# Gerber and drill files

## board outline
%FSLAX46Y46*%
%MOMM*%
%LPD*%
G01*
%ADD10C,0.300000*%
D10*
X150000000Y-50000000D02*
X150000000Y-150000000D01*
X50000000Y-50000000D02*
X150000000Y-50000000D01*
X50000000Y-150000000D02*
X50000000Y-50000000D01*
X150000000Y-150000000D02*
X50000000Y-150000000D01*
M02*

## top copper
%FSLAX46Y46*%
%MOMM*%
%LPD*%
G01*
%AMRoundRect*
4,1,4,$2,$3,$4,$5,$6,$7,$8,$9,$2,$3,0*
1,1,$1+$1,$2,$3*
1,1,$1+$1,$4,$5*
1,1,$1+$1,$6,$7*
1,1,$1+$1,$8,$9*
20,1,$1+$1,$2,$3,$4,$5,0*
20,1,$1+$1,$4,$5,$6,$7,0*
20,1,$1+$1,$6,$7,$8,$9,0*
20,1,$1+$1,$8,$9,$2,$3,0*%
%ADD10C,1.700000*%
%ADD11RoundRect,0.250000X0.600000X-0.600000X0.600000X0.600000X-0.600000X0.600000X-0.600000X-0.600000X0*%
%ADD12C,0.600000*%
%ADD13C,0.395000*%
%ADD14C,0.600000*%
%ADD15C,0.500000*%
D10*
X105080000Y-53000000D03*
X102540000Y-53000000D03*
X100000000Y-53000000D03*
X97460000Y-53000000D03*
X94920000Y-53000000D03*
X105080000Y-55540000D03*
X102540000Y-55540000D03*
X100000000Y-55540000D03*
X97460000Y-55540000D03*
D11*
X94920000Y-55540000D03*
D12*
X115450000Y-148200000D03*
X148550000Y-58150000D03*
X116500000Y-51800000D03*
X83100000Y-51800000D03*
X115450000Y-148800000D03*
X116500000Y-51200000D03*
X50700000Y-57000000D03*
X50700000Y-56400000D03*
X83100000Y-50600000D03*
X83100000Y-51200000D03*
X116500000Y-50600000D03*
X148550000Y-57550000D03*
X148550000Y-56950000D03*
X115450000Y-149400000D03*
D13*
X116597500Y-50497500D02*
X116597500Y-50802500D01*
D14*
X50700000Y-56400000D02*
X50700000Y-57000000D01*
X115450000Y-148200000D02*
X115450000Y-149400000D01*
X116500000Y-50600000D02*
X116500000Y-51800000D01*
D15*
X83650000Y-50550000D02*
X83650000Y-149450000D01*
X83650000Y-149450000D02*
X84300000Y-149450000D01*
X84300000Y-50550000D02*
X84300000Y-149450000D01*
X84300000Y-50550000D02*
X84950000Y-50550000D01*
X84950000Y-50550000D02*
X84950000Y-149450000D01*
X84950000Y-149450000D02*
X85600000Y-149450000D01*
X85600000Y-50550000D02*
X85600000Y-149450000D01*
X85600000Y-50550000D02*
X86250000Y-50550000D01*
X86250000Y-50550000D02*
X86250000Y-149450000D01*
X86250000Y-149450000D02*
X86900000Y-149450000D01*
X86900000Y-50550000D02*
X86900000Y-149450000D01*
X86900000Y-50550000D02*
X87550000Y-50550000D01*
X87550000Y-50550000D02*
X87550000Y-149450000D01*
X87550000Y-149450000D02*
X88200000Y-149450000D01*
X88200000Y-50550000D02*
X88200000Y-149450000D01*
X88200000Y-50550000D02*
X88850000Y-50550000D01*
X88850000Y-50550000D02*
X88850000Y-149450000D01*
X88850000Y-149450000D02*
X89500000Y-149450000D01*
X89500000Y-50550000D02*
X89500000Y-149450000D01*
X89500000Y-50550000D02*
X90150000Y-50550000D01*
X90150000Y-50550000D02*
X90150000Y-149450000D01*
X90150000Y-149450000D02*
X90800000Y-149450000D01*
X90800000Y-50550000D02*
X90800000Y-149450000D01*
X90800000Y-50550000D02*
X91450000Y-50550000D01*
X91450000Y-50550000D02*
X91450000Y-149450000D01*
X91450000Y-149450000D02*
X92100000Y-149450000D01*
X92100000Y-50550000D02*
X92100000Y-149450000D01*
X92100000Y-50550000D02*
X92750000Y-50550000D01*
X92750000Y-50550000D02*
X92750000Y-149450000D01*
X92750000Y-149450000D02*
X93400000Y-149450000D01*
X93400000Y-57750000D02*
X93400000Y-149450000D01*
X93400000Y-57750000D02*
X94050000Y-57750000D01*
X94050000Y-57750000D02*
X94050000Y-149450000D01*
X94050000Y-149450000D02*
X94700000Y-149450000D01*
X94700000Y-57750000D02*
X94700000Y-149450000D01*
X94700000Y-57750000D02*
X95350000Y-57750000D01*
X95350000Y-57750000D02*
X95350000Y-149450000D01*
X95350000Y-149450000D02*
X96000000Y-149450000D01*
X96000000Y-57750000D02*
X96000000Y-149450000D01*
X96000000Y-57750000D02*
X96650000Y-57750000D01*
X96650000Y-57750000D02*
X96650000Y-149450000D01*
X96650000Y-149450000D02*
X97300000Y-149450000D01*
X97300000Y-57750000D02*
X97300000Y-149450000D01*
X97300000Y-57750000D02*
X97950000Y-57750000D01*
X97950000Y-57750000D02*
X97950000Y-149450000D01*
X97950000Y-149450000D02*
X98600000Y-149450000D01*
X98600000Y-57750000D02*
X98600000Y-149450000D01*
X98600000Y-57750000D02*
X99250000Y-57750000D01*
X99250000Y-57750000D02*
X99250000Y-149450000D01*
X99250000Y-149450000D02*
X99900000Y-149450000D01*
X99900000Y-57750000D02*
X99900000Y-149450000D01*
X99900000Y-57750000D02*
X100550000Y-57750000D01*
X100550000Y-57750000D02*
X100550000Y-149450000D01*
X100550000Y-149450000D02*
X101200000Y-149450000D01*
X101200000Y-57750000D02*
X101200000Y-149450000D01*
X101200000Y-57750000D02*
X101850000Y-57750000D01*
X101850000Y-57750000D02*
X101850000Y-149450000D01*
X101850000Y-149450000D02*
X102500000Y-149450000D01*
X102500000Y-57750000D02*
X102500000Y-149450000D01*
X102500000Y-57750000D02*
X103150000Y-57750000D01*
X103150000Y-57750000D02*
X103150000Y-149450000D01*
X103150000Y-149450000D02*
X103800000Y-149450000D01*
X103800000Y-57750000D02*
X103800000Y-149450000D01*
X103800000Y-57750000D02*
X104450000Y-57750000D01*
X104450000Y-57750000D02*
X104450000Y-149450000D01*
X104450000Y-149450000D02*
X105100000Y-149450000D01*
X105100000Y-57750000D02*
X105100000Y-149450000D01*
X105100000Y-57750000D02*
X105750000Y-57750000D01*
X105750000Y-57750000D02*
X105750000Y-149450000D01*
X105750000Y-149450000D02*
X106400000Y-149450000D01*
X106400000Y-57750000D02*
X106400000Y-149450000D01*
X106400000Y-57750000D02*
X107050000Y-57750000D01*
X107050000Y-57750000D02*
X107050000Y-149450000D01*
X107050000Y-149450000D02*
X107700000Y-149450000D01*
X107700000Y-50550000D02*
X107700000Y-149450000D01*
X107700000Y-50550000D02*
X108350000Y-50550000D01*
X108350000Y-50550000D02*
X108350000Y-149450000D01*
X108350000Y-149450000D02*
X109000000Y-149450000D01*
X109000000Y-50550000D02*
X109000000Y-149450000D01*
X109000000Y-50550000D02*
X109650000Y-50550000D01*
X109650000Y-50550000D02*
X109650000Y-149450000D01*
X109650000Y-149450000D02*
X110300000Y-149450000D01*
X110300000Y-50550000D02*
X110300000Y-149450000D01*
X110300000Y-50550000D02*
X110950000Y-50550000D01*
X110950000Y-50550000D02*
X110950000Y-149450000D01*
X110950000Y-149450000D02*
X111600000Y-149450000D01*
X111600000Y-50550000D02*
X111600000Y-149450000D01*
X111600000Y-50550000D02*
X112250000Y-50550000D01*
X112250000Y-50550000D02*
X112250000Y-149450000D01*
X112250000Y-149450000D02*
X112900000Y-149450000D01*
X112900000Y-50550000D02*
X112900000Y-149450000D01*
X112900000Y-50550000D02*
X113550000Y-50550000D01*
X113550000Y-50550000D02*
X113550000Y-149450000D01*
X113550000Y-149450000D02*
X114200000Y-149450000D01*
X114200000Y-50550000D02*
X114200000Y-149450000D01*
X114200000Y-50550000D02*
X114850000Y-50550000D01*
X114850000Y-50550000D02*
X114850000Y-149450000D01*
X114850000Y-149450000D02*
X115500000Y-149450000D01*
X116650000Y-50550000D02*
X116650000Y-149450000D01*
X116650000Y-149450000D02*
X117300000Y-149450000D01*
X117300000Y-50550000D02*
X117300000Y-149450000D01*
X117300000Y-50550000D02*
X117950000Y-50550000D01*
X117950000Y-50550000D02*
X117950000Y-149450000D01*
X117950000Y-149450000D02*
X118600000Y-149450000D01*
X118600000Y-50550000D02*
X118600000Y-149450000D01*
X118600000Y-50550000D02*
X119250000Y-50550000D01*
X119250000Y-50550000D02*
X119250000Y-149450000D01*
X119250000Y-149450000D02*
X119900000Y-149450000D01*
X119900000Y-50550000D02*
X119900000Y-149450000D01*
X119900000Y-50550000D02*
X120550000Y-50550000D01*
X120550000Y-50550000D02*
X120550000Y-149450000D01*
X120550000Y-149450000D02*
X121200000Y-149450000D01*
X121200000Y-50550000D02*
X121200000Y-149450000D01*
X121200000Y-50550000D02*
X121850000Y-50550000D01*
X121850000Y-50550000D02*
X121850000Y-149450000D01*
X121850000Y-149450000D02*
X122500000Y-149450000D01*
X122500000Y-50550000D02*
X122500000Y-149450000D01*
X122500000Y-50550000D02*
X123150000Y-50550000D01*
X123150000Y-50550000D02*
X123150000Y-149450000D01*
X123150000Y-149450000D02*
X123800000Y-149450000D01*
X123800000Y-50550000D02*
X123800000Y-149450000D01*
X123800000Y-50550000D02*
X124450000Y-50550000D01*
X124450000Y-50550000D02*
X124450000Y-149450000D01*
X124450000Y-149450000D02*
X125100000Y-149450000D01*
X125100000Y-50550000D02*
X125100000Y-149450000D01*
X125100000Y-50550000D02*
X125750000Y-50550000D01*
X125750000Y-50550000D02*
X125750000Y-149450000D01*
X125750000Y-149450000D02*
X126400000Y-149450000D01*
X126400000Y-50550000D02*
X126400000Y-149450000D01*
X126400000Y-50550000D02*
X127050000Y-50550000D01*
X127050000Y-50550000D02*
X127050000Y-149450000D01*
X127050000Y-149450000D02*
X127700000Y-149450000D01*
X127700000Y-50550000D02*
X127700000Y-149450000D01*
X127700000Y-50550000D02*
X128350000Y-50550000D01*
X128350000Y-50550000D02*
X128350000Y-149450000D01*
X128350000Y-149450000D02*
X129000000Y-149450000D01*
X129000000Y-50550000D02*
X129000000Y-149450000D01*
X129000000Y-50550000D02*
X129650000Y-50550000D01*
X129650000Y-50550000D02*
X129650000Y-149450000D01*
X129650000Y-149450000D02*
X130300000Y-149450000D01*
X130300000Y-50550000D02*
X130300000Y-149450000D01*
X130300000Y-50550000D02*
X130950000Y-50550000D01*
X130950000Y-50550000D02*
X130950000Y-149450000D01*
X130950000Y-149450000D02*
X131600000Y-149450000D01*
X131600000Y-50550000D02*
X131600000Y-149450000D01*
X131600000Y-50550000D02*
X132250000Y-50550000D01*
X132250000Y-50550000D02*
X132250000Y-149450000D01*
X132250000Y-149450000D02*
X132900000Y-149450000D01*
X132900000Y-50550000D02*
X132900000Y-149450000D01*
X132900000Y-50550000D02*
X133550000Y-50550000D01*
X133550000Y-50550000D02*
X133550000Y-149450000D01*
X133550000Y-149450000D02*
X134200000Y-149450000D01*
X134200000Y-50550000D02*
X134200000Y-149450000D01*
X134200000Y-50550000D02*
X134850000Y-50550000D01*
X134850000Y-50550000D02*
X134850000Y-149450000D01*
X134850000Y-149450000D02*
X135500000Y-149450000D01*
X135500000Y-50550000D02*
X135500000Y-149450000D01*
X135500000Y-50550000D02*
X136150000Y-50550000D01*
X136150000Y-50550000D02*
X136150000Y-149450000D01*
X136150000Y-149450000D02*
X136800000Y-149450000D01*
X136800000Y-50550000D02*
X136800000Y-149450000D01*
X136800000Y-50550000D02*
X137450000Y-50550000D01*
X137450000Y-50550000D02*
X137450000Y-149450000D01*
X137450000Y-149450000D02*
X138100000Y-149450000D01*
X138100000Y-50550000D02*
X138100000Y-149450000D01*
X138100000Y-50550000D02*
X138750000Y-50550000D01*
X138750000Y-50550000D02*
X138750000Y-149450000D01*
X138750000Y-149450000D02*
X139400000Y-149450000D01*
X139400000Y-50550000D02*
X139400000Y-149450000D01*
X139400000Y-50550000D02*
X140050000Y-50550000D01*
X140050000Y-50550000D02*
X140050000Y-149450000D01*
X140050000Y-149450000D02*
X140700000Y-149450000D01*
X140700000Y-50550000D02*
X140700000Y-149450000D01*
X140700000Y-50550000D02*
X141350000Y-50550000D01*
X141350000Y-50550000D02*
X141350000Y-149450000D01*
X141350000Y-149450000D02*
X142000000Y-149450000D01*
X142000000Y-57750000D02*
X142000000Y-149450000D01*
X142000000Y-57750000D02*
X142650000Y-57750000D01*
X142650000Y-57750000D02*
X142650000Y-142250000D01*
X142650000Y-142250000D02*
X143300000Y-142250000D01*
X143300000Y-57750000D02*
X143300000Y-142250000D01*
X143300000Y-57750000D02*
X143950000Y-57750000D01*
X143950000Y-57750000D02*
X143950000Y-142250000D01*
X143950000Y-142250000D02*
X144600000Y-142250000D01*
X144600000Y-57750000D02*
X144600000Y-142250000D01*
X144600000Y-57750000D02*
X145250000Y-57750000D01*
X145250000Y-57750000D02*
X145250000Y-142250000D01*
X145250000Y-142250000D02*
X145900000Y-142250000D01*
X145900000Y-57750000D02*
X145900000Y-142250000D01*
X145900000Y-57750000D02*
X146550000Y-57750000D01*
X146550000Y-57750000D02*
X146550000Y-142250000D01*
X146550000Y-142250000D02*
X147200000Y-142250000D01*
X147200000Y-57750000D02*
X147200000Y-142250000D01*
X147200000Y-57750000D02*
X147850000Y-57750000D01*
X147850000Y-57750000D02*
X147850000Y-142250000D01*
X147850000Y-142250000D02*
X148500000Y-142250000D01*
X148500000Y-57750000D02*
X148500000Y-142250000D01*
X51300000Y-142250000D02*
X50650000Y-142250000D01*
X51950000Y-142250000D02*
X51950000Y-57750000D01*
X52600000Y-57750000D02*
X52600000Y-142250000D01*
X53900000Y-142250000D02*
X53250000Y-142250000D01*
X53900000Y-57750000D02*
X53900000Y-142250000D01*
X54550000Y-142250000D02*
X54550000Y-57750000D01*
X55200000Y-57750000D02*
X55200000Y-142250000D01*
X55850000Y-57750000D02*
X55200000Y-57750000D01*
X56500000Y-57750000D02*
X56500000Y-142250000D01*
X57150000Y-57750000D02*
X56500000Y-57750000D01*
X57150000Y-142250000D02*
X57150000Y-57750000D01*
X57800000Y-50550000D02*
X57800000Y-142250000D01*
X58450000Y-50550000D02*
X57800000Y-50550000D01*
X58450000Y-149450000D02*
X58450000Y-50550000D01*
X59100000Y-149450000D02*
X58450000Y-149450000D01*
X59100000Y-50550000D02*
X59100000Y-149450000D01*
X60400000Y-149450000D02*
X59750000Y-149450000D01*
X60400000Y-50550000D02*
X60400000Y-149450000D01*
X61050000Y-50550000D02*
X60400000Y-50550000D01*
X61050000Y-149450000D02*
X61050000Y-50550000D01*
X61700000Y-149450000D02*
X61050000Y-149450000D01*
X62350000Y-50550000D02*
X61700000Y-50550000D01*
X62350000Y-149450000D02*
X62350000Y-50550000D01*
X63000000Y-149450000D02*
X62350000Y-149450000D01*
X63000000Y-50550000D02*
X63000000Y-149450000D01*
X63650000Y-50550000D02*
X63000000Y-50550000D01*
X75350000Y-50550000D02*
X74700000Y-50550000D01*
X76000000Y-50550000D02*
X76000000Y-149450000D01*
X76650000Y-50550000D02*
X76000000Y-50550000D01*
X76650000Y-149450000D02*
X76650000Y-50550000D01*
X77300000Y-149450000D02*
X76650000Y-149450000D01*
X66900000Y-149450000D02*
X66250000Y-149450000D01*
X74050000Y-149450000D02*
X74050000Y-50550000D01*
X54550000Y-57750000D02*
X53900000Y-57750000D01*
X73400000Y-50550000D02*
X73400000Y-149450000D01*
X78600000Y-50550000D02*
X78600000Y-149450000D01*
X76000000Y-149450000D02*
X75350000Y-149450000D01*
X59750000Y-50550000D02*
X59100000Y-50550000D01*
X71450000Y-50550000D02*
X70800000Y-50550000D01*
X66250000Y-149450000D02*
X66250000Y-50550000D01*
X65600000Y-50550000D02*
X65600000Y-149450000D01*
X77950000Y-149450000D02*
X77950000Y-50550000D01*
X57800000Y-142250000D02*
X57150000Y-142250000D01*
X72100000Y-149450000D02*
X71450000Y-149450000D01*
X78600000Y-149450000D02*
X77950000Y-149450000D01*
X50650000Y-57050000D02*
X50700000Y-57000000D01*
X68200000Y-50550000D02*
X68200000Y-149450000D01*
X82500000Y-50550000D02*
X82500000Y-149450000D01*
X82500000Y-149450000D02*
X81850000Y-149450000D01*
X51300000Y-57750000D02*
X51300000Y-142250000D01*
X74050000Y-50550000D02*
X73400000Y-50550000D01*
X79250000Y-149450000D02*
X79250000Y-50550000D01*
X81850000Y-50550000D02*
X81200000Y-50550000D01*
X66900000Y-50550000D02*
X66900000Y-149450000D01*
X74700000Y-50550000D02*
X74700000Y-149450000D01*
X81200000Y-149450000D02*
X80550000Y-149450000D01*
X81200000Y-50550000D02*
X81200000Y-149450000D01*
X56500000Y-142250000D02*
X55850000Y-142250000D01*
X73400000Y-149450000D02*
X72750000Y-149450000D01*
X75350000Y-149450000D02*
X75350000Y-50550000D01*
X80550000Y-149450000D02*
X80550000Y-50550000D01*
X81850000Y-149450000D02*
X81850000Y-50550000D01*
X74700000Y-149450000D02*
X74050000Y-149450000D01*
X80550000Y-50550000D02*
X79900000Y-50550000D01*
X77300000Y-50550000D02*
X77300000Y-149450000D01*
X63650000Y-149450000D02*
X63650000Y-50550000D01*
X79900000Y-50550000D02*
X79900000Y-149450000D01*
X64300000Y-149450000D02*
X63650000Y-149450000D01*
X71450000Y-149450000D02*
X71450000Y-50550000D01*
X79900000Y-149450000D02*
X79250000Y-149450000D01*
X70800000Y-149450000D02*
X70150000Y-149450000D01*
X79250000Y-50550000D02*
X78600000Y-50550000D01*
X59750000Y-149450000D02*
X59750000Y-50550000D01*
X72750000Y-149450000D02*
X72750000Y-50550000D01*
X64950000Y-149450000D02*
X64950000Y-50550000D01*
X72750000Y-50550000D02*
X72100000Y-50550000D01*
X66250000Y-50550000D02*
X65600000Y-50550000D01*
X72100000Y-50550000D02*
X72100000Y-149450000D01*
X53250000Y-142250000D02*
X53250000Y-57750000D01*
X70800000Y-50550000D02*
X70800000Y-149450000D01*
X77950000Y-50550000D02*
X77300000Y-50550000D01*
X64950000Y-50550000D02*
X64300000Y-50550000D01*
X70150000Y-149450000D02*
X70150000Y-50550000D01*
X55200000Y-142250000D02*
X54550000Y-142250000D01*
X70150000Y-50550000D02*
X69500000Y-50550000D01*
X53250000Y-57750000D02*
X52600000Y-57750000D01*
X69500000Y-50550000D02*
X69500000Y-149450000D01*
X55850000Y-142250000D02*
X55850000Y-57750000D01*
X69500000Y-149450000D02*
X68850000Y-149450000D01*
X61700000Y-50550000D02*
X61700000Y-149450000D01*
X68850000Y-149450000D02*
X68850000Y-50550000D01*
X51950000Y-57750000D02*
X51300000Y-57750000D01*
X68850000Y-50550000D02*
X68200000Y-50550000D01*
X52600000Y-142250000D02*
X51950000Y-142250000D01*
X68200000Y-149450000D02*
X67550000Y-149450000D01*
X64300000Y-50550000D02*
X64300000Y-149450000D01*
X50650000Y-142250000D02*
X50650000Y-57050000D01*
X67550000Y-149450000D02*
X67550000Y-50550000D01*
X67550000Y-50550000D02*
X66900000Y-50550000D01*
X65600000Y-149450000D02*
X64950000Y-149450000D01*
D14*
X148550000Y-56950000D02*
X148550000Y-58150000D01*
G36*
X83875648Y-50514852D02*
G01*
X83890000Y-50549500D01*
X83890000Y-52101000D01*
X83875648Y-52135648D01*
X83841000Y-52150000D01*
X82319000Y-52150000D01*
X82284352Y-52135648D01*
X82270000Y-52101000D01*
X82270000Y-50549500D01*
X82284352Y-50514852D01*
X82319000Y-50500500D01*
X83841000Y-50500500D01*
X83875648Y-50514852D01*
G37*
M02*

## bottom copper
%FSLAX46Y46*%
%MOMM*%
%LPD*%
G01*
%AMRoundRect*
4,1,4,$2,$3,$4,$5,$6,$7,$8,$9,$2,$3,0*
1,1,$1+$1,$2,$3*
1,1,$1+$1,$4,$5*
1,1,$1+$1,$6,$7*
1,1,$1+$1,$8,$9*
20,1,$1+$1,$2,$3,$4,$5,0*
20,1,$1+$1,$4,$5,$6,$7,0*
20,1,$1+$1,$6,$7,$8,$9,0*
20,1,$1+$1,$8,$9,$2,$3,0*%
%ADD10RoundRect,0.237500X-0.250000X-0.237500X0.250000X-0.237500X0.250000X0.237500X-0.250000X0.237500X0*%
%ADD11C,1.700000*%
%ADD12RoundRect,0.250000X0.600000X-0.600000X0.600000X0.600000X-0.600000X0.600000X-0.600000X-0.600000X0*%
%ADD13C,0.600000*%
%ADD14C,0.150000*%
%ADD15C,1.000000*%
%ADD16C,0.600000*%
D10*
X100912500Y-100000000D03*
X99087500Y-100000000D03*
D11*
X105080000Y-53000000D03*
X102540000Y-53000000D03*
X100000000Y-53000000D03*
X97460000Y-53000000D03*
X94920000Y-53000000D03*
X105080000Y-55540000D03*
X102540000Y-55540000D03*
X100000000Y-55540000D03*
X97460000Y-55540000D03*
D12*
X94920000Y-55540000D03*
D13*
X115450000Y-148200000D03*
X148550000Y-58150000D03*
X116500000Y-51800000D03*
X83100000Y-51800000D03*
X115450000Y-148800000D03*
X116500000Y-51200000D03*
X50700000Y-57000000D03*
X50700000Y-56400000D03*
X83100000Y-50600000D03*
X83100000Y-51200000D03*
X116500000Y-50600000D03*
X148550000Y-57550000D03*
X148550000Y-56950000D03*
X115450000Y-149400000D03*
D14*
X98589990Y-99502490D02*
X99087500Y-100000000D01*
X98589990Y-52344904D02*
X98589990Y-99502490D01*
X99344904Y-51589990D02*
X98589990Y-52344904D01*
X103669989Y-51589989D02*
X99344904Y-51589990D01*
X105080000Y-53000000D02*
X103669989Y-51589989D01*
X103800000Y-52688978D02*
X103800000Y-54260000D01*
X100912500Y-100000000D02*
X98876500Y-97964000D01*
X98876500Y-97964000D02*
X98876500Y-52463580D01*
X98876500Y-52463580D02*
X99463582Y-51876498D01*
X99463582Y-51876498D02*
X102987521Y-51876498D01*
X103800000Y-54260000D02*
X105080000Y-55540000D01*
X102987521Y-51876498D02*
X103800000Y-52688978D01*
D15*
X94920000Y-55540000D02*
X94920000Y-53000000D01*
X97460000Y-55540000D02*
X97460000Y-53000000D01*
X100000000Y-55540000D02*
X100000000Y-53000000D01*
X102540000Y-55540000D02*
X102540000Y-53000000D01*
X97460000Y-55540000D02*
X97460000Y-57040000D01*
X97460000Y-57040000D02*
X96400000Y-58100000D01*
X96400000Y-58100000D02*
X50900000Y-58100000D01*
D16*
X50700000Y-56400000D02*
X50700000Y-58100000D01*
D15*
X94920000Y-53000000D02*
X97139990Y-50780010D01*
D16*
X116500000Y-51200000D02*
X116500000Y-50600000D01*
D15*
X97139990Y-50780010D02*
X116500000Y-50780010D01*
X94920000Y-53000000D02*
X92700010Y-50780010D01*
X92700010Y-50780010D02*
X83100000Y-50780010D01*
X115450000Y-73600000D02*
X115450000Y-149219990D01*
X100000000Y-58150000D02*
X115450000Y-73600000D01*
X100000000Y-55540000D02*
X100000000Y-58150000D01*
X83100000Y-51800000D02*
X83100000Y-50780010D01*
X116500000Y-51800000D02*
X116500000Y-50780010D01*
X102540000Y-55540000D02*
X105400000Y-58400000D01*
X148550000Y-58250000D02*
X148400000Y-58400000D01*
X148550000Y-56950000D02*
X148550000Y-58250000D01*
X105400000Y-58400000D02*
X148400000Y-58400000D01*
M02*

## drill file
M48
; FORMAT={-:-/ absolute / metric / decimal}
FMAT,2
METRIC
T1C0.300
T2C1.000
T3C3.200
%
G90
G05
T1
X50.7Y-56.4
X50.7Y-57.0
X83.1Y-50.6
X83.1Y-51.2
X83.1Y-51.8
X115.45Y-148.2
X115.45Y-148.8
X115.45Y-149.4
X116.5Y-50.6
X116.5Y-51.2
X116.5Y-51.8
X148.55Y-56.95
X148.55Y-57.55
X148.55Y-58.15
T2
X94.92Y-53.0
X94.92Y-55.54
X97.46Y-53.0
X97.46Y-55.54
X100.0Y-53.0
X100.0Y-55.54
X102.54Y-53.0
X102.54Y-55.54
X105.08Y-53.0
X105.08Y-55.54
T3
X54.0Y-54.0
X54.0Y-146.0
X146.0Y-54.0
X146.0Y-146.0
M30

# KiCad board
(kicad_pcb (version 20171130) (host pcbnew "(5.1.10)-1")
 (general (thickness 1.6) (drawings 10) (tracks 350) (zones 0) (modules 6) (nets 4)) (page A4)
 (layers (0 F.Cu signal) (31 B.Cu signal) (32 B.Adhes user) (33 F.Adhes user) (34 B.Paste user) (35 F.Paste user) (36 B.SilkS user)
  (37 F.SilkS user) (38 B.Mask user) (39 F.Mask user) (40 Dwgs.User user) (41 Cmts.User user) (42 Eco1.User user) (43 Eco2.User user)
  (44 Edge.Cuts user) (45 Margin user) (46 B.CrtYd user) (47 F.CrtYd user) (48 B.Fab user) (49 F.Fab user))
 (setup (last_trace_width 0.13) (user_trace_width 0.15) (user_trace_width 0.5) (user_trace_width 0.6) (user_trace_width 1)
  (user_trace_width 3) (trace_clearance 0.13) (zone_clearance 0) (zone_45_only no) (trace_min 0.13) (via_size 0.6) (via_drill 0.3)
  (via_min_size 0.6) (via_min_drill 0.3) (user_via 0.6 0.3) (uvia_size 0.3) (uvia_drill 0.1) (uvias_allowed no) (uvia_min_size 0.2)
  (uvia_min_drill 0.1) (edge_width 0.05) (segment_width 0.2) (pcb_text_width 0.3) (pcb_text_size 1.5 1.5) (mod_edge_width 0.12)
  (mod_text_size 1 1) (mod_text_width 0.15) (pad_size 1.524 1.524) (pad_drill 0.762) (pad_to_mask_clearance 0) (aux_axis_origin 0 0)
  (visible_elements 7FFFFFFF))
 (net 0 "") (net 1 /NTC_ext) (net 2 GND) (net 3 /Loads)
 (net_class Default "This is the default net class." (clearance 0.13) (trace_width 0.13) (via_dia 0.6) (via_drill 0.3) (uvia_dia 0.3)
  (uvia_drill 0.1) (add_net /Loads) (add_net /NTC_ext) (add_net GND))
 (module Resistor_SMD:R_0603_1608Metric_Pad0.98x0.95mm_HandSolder (layer B.Cu) (at 100 100)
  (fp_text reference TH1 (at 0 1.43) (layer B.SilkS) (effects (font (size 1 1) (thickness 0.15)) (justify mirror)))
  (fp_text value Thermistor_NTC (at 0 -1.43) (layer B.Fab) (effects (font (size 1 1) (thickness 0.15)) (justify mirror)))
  (pad 2 smd roundrect (at 0.9125 0) (size 0.975 0.95) (layers B.Cu B.Paste B.Mask) (roundrect_rratio 0.25) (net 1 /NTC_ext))
  (pad 1 smd roundrect (at -0.9125 0) (size 0.975 0.95) (layers B.Cu B.Paste B.Mask) (roundrect_rratio 0.25) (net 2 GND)))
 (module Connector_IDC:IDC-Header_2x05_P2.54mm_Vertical (layer F.Cu) (at 94.92 55.54 90)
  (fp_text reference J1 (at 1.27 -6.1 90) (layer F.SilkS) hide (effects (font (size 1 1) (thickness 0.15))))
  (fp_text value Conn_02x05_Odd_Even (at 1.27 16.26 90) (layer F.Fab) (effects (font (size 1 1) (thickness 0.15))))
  (pad 10 thru_hole circle (at 2.54 10.16 90) (size 1.7 1.7) (drill 1) (layers *.Cu *.Mask) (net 2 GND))
  (pad 8 thru_hole circle (at 2.54 7.62 90) (size 1.7 1.7) (drill 1) (layers *.Cu *.Mask) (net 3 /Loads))
  (pad 6 thru_hole circle (at 2.54 5.08 90) (size 1.7 1.7) (drill 1) (layers *.Cu *.Mask) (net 3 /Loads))
  (pad 4 thru_hole circle (at 2.54 2.54 90) (size 1.7 1.7) (drill 1) (layers *.Cu *.Mask) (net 3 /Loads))
  (pad 2 thru_hole circle (at 2.54 0 90) (size 1.7 1.7) (drill 1) (layers *.Cu *.Mask) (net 3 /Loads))
  (pad 9 thru_hole circle (at 0 10.16 90) (size 1.7 1.7) (drill 1) (layers *.Cu *.Mask) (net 1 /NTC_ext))
  (pad 7 thru_hole circle (at 0 7.62 90) (size 1.7 1.7) (drill 1) (layers *.Cu *.Mask) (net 3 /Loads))
  (pad 5 thru_hole circle (at 0 5.08 90) (size 1.7 1.7) (drill 1) (layers *.Cu *.Mask) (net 3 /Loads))
  (pad 3 thru_hole circle (at 0 2.54 90) (size 1.7 1.7) (drill 1) (layers *.Cu *.Mask) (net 3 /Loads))
  (pad 1 thru_hole roundrect (at 0 0 90) (size 1.7 1.7) (drill 1) (layers *.Cu *.Mask) (roundrect_rratio 0.1470588235294118) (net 3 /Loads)))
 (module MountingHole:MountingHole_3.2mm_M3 (layer F.Cu) (at 146 146)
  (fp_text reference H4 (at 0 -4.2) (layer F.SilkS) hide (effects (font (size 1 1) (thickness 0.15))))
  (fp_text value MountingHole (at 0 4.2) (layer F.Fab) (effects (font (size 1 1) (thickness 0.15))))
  (pad 1 np_thru_hole circle (at 0 0) (size 3.2 3.2) (drill 3.2) (layers *.Cu *.Mask)))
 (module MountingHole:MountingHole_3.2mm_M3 (layer F.Cu) (at 54 146)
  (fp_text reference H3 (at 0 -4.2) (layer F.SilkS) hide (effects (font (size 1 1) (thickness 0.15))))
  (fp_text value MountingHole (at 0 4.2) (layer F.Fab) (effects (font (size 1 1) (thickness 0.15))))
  (pad 1 np_thru_hole circle (at 0 0) (size 3.2 3.2) (drill 3.2) (layers *.Cu *.Mask)))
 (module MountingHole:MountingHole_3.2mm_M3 (layer F.Cu) (at 146 54)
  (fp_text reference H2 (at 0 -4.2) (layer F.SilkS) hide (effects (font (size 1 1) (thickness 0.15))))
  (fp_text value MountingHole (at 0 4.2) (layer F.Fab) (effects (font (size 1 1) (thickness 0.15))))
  (pad 1 np_thru_hole circle (at 0 0) (size 3.2 3.2) (drill 3.2) (layers *.Cu *.Mask)))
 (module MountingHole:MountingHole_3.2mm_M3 (layer F.Cu) (at 54 54)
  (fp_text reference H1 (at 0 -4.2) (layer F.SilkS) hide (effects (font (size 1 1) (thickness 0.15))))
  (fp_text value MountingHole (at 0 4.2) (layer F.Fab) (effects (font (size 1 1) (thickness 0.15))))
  (pad 1 np_thru_hole circle (at 0 0) (size 3.2 3.2) (drill 3.2) (layers *.Cu *.Mask)))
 (gr_line (start 150 50) (end 150 150) (layer Edge.Cuts) (width 0.3))
 (gr_line (start 50 50) (end 150 50) (layer Edge.Cuts) (width 0.3))
 (gr_line (start 50 150) (end 50 50) (layer Edge.Cuts) (width 0.3))
 (gr_line (start 150 150) (end 50 150) (layer Edge.Cuts) (width 0.3))
 (segment (start 98.58999 99.50249) (end 99.0875 100) (width 0.15) (layer B.Cu) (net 2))
 (segment (start 98.58999 52.344904) (end 98.58999 99.50249) (width 0.15) (layer B.Cu) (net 2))
 (segment (start 99.344904 51.58999) (end 98.58999 52.344904) (width 0.15) (layer B.Cu) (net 2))
 (segment (start 103.669989 51.589989) (end 99.344904 51.58999) (width 0.15) (layer B.Cu) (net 2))
 (segment (start 105.08 53) (end 103.669989 51.589989) (width 0.15) (layer B.Cu) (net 2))
 (segment (start 103.8 52.688978) (end 103.8 54.26) (width 0.15) (layer B.Cu) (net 1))
 (segment (start 100.9125 100) (end 98.8765 97.964) (width 0.15) (layer B.Cu) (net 1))
 (segment (start 98.8765 97.964) (end 98.8765 52.46358) (width 0.15) (layer B.Cu) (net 1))
 (segment (start 98.8765 52.46358) (end 99.463582 51.876498) (width 0.15) (layer B.Cu) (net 1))
 (segment (start 99.463582 51.876498) (end 102.987521 51.876498) (width 0.15) (layer B.Cu) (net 1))
 (segment (start 103.8 54.26) (end 105.08 55.54) (width 0.15) (layer B.Cu) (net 1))
 (segment (start 102.987521 51.876498) (end 103.8 52.688978) (width 0.15) (layer B.Cu) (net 1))
 (via (at 115.45 148.2) (size 0.6) (drill 0.3) (layers F.Cu B.Cu) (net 3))
 (via (at 148.55 58.15) (size 0.6) (drill 0.3) (layers F.Cu B.Cu) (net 3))
 (via (at 116.5 51.8) (size 0.6) (drill 0.3) (layers F.Cu B.Cu) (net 3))
 (via (at 83.1 51.8) (size 0.6) (drill 0.3) (layers F.Cu B.Cu) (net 3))
 (via (at 115.45 148.8) (size 0.6) (drill 0.3) (layers F.Cu B.Cu) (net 3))
 (via (at 116.5 51.2) (size 0.6) (drill 0.3) (layers F.Cu B.Cu) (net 3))
 (via (at 50.7 57) (size 0.6) (drill 0.3) (layers F.Cu B.Cu) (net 3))
 (via (at 50.7 56.4) (size 0.6) (drill 0.3) (layers F.Cu B.Cu) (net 3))
 (segment (start 94.92 55.54) (end 94.92 53) (width 1) (layer B.Cu) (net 3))
 (segment (start 97.46 55.54) (end 97.46 53) (width 1) (layer B.Cu) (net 3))
 (segment (start 100 55.54) (end 100 53) (width 1) (layer B.Cu) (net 3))
 (segment (start 102.54 55.54) (end 102.54 53) (width 1) (layer B.Cu) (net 3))
 (segment (start 116.5975 50.4975) (end 116.5975 50.8025) (width 0.395) (layer F.Cu) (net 3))
 (via (at 83.1 50.6) (size 0.6) (drill 0.3) (layers F.Cu B.Cu) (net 3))
 (via (at 83.1 51.2) (size 0.6) (drill 0.3) (layers F.Cu B.Cu) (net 3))
 (segment (start 97.46 55.54) (end 97.46 57.04) (width 1) (layer B.Cu) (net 3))
 (segment (start 97.46 57.04) (end 96.4 58.1) (width 1) (layer B.Cu) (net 3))
 (segment (start 96.4 58.1) (end 50.9 58.1) (width 1) (layer B.Cu) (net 3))
 (segment (start 50.7 56.4) (end 50.7 58.1) (width 0.6) (layer B.Cu) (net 3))
 (segment (start 50.7 56.4) (end 50.7 57) (width 0.6) (layer F.Cu) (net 3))
 (via (at 116.5 50.6) (size 0.6) (drill 0.3) (layers F.Cu B.Cu) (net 3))
 (segment (start 94.92 53) (end 97.13999 50.78001) (width 1) (layer B.Cu) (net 3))
 (segment (start 116.5 51.2) (end 116.5 50.6) (width 0.6) (layer B.Cu) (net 3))
 (segment (start 97.13999 50.78001) (end 116.5 50.78001) (width 1) (layer B.Cu) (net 3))
 (segment (start 94.92 53) (end 92.70001 50.78001) (width 1) (layer B.Cu) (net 3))
 (segment (start 92.70001 50.78001) (end 83.1 50.78001) (width 1) (layer B.Cu) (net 3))
 (via (at 148.55 57.55) (size 0.6) (drill 0.3) (layers F.Cu B.Cu) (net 3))
 (via (at 148.55 56.95) (size 0.6) (drill 0.3) (layers F.Cu B.Cu) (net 3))
 (via (at 115.45 149.4) (size 0.6) (drill 0.3) (layers F.Cu B.Cu) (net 3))
 (segment (start 115.45 73.6) (end 115.45 149.21999) (width 1) (layer B.Cu) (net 3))
 (segment (start 100 58.15) (end 115.45 73.6) (width 1) (layer B.Cu) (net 3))
 (segment (start 100 55.54) (end 100 58.15) (width 1) (layer B.Cu) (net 3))
 (segment (start 83.1 51.8) (end 83.1 50.78001) (width 1) (layer B.Cu) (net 3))
 (segment (start 116.5 51.8) (end 116.5 50.78001) (width 1) (layer B.Cu) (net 3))
 (segment (start 102.54 55.54) (end 105.4 58.4) (width 1) (layer B.Cu) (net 3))
 (segment (start 115.45 148.2) (end 115.45 149.4) (width 0.6) (layer F.Cu) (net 3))
 (segment (start 116.5 50.6) (end 116.5 51.8) (width 0.6) (layer F.Cu) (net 3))
 (segment (start 83.65 50.55) (end 83.65 149.45) (width 0.5) (layer F.Cu) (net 3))
 (segment (start 83.65 149.45) (end 84.3 149.45) (width 0.5) (layer F.Cu) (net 3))
 (segment (start 84.3 50.55) (end 84.3 149.45) (width 0.5) (layer F.Cu) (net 3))
 (segment (start 84.3 50.55) (end 84.95 50.55) (width 0.5) (layer F.Cu) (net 3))
 (segment (start 84.95 50.55) (end 84.95 149.45) (width 0.5) (layer F.Cu) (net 3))
 (segment (start 84.95 149.45) (end 85.6 149.45) (width 0.5) (layer F.Cu) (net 3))
 (segment (start 85.6 50.55) (end 85.6 149.45) (width 0.5) (layer F.Cu) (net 3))
 (segment (start 85.6 50.55) (end 86.25 50.55) (width 0.5) (layer F.Cu) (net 3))
 (segment (start 86.25 50.55) (end 86.25 149.45) (width 0.5) (layer F.Cu) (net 3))
 (segment (start 86.25 149.45) (end 86.9 149.45) (width 0.5) (layer F.Cu) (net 3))
 (segment (start 86.9 50.55) (end 86.9 149.45) (width 0.5) (layer F.Cu) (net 3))
 (segment (start 86.9 50.55) (end 87.55 50.55) (width 0.5) (layer F.Cu) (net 3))
 (segment (start 87.55 50.55) (end 87.55 149.45) (width 0.5) (layer F.Cu) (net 3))
 (segment (start 87.55 149.45) (end 88.2 149.45) (width 0.5) (layer F.Cu) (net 3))
 (segment (start 88.2 50.55) (end 88.2 149.45) (width 0.5) (layer F.Cu) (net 3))
 (segment (start 88.2 50.55) (end 88.85 50.55) (width 0.5) (layer F.Cu) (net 3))
 (segment (start 88.85 50.55) (end 88.85 149.45) (width 0.5) (layer F.Cu) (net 3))
 (segment (start 88.85 149.45) (end 89.5 149.45) (width 0.5) (layer F.Cu) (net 3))
 (segment (start 89.5 50.55) (end 89.5 149.45) (width 0.5) (layer F.Cu) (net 3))
 (segment (start 89.5 50.55) (end 90.15 50.55) (width 0.5) (layer F.Cu) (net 3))
 (segment (start 90.15 50.55) (end 90.15 149.45) (width 0.5) (layer F.Cu) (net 3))
 (segment (start 90.15 149.45) (end 90.8 149.45) (width 0.5) (layer F.Cu) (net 3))
 (segment (start 90.8 50.55) (end 90.8 149.45) (width 0.5) (layer F.Cu) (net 3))
 (segment (start 90.8 50.55) (end 91.45 50.55) (width 0.5) (layer F.Cu) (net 3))
 (segment (start 91.45 50.55) (end 91.45 149.45) (width 0.5) (layer F.Cu) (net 3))
 (segment (start 91.45 149.45) (end 92.1 149.45) (width 0.5) (layer F.Cu) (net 3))
 (segment (start 92.1 50.55) (end 92.1 149.45) (width 0.5) (layer F.Cu) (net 3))
 (segment (start 92.1 50.55) (end 92.75 50.55) (width 0.5) (layer F.Cu) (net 3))
 (segment (start 92.75 50.55) (end 92.75 149.45) (width 0.5) (layer F.Cu) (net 3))
 (segment (start 92.75 149.45) (end 93.4 149.45) (width 0.5) (layer F.Cu) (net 3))
 (segment (start 93.4 57.75) (end 93.4 149.45) (width 0.5) (layer F.Cu) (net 3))
 (segment (start 93.4 57.75) (end 94.05 57.75) (width 0.5) (layer F.Cu) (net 3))
 (segment (start 94.05 57.75) (end 94.05 149.45) (width 0.5) (layer F.Cu) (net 3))
 (segment (start 94.05 149.45) (end 94.7 149.45) (width 0.5) (layer F.Cu) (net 3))
 (segment (start 94.7 57.75) (end 94.7 149.45) (width 0.5) (layer F.Cu) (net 3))
 (segment (start 94.7 57.75) (end 95.35 57.75) (width 0.5) (layer F.Cu) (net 3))
 (segment (start 95.35 57.75) (end 95.35 149.45) (width 0.5) (layer F.Cu) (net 3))
 (segment (start 95.35 149.45) (end 96 149.45) (width 0.5) (layer F.Cu) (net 3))
 (segment (start 96 57.75) (end 96 149.45) (width 0.5) (layer F.Cu) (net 3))
 (segment (start 96 57.75) (end 96.65 57.75) (width 0.5) (layer F.Cu) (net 3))
 (segment (start 96.65 57.75) (end 96.65 149.45) (width 0.5) (layer F.Cu) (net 3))
 (segment (start 96.65 149.45) (end 97.3 149.45) (width 0.5) (layer F.Cu) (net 3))
 (segment (start 97.3 57.75) (end 97.3 149.45) (width 0.5) (layer F.Cu) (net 3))
 (segment (start 97.3 57.75) (end 97.95 57.75) (width 0.5) (layer F.Cu) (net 3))
 (segment (start 97.95 57.75) (end 97.95 149.45) (width 0.5) (layer F.Cu) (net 3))
 (segment (start 97.95 149.45) (end 98.6 149.45) (width 0.5) (layer F.Cu) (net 3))
 (segment (start 98.6 57.75) (end 98.6 149.45) (width 0.5) (layer F.Cu) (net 3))
 (segment (start 98.6 57.75) (end 99.25 57.75) (width 0.5) (layer F.Cu) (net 3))
 (segment (start 99.25 57.75) (end 99.25 149.45) (width 0.5) (layer F.Cu) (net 3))
 (segment (start 99.25 149.45) (end 99.9 149.45) (width 0.5) (layer F.Cu) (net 3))
 (segment (start 99.9 57.75) (end 99.9 149.45) (width 0.5) (layer F.Cu) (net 3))
 (segment (start 99.9 57.75) (end 100.55 57.75) (width 0.5) (layer F.Cu) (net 3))
 (segment (start 100.55 57.75) (end 100.55 149.45) (width 0.5) (layer F.Cu) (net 3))
 (segment (start 100.55 149.45) (end 101.2 149.45) (width 0.5) (layer F.Cu) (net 3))
 (segment (start 101.2 57.75) (end 101.2 149.45) (width 0.5) (layer F.Cu) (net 3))
 (segment (start 101.2 57.75) (end 101.85 57.75) (width 0.5) (layer F.Cu) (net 3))
 (segment (start 101.85 57.75) (end 101.85 149.45) (width 0.5) (layer F.Cu) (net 3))
 (segment (start 101.85 149.45) (end 102.5 149.45) (width 0.5) (layer F.Cu) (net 3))
 (segment (start 102.5 57.75) (end 102.5 149.45) (width 0.5) (layer F.Cu) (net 3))
 (segment (start 102.5 57.75) (end 103.15 57.75) (width 0.5) (layer F.Cu) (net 3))
 (segment (start 103.15 57.75) (end 103.15 149.45) (width 0.5) (layer F.Cu) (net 3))
 (segment (start 103.15 149.45) (end 103.8 149.45) (width 0.5) (layer F.Cu) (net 3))
 (segment (start 103.8 57.75) (end 103.8 149.45) (width 0.5) (layer F.Cu) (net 3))
 (segment (start 103.8 57.75) (end 104.45 57.75) (width 0.5) (layer F.Cu) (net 3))
 (segment (start 104.45 57.75) (end 104.45 149.45) (width 0.5) (layer F.Cu) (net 3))
 (segment (start 104.45 149.45) (end 105.1 149.45) (width 0.5) (layer F.Cu) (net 3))
 (segment (start 105.1 57.75) (end 105.1 149.45) (width 0.5) (layer F.Cu) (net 3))
 (segment (start 105.1 57.75) (end 105.75 57.75) (width 0.5) (layer F.Cu) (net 3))
 (segment (start 105.75 57.75) (end 105.75 149.45) (width 0.5) (layer F.Cu) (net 3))
 (segment (start 105.75 149.45) (end 106.4 149.45) (width 0.5) (layer F.Cu) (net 3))
 (segment (start 106.4 57.75) (end 106.4 149.45) (width 0.5) (layer F.Cu) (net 3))
 (segment (start 106.4 57.75) (end 107.05 57.75) (width 0.5) (layer F.Cu) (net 3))
 (segment (start 107.05 57.75) (end 107.05 149.45) (width 0.5) (layer F.Cu) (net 3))
 (segment (start 107.05 149.45) (end 107.7 149.45) (width 0.5) (layer F.Cu) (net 3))
 (segment (start 107.7 50.55) (end 107.7 149.45) (width 0.5) (layer F.Cu) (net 3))
 (segment (start 107.7 50.55) (end 108.35 50.55) (width 0.5) (layer F.Cu) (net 3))
 (segment (start 108.35 50.55) (end 108.35 149.45) (width 0.5) (layer F.Cu) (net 3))
 (segment (start 108.35 149.45) (end 109 149.45) (width 0.5) (layer F.Cu) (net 3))
 (segment (start 109 50.55) (end 109 149.45) (width 0.5) (layer F.Cu) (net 3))
 (segment (start 109 50.55) (end 109.65 50.55) (width 0.5) (layer F.Cu) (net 3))
 (segment (start 109.65 50.55) (end 109.65 149.45) (width 0.5) (layer F.Cu) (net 3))
 (segment (start 109.65 149.45) (end 110.3 149.45) (width 0.5) (layer F.Cu) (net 3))
 (segment (start 110.3 50.55) (end 110.3 149.45) (width 0.5) (layer F.Cu) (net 3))
 (segment (start 110.3 50.55) (end 110.95 50.55) (width 0.5) (layer F.Cu) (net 3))
 (segment (start 110.95 50.55) (end 110.95 149.45) (width 0.5) (layer F.Cu) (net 3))
 (segment (start 110.95 149.45) (end 111.6 149.45) (width 0.5) (layer F.Cu) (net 3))
 (segment (start 111.6 50.55) (end 111.6 149.45) (width 0.5) (layer F.Cu) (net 3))
 (segment (start 111.6 50.55) (end 112.25 50.55) (width 0.5) (layer F.Cu) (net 3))
 (segment (start 112.25 50.55) (end 112.25 149.45) (width 0.5) (layer F.Cu) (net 3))
 (segment (start 112.25 149.45) (end 112.9 149.45) (width 0.5) (layer F.Cu) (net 3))
 (segment (start 112.9 50.55) (end 112.9 149.45) (width 0.5) (layer F.Cu) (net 3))
 (segment (start 112.9 50.55) (end 113.55 50.55) (width 0.5) (layer F.Cu) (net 3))
 (segment (start 113.55 50.55) (end 113.55 149.45) (width 0.5) (layer F.Cu) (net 3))
 (segment (start 113.55 149.45) (end 114.2 149.45) (width 0.5) (layer F.Cu) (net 3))
 (segment (start 114.2 50.55) (end 114.2 149.45) (width 0.5) (layer F.Cu) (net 3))
 (segment (start 114.2 50.55) (end 114.85 50.55) (width 0.5) (layer F.Cu) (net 3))
 (segment (start 114.85 50.55) (end 114.85 149.45) (width 0.5) (layer F.Cu) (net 3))
 (segment (start 114.85 149.45) (end 115.5 149.45) (width 0.5) (layer F.Cu) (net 3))
 (segment (start 116.65 50.55) (end 116.65 149.45) (width 0.5) (layer F.Cu) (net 3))
 (segment (start 116.65 149.45) (end 117.3 149.45) (width 0.5) (layer F.Cu) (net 3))
 (segment (start 117.3 50.55) (end 117.3 149.45) (width 0.5) (layer F.Cu) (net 3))
 (segment (start 117.3 50.55) (end 117.95 50.55) (width 0.5) (layer F.Cu) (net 3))
 (segment (start 117.95 50.55) (end 117.95 149.45) (width 0.5) (layer F.Cu) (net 3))
 (segment (start 117.95 149.45) (end 118.6 149.45) (width 0.5) (layer F.Cu) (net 3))
 (segment (start 118.6 50.55) (end 118.6 149.45) (width 0.5) (layer F.Cu) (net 3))
 (segment (start 118.6 50.55) (end 119.25 50.55) (width 0.5) (layer F.Cu) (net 3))
 (segment (start 119.25 50.55) (end 119.25 149.45) (width 0.5) (layer F.Cu) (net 3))
 (segment (start 119.25 149.45) (end 119.9 149.45) (width 0.5) (layer F.Cu) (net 3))
 (segment (start 119.9 50.55) (end 119.9 149.45) (width 0.5) (layer F.Cu) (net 3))
 (segment (start 119.9 50.55) (end 120.55 50.55) (width 0.5) (layer F.Cu) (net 3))
 (segment (start 120.55 50.55) (end 120.55 149.45) (width 0.5) (layer F.Cu) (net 3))
 (segment (start 120.55 149.45) (end 121.2 149.45) (width 0.5) (layer F.Cu) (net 3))
 (segment (start 121.2 50.55) (end 121.2 149.45) (width 0.5) (layer F.Cu) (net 3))
 (segment (start 121.2 50.55) (end 121.85 50.55) (width 0.5) (layer F.Cu) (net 3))
 (segment (start 121.85 50.55) (end 121.85 149.45) (width 0.5) (layer F.Cu) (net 3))
 (segment (start 121.85 149.45) (end 122.5 149.45) (width 0.5) (layer F.Cu) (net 3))
 (segment (start 122.5 50.55) (end 122.5 149.45) (width 0.5) (layer F.Cu) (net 3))
 (segment (start 122.5 50.55) (end 123.15 50.55) (width 0.5) (layer F.Cu) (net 3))
 (segment (start 123.15 50.55) (end 123.15 149.45) (width 0.5) (layer F.Cu) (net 3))
 (segment (start 123.15 149.45) (end 123.8 149.45) (width 0.5) (layer F.Cu) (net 3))
 (segment (start 123.8 50.55) (end 123.8 149.45) (width 0.5) (layer F.Cu) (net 3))
 (segment (start 123.8 50.55) (end 124.45 50.55) (width 0.5) (layer F.Cu) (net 3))
 (segment (start 124.45 50.55) (end 124.45 149.45) (width 0.5) (layer F.Cu) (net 3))
 (segment (start 124.45 149.45) (end 125.1 149.45) (width 0.5) (layer F.Cu) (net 3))
 (segment (start 125.1 50.55) (end 125.1 149.45) (width 0.5) (layer F.Cu) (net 3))
 (segment (start 125.1 50.55) (end 125.75 50.55) (width 0.5) (layer F.Cu) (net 3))
 (segment (start 125.75 50.55) (end 125.75 149.45) (width 0.5) (layer F.Cu) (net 3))
 (segment (start 125.75 149.45) (end 126.4 149.45) (width 0.5) (layer F.Cu) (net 3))
 (segment (start 126.4 50.55) (end 126.4 149.45) (width 0.5) (layer F.Cu) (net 3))
 (segment (start 126.4 50.55) (end 127.05 50.55) (width 0.5) (layer F.Cu) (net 3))
 (segment (start 127.05 50.55) (end 127.05 149.45) (width 0.5) (layer F.Cu) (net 3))
 (segment (start 127.05 149.45) (end 127.7 149.45) (width 0.5) (layer F.Cu) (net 3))
 (segment (start 127.7 50.55) (end 127.7 149.45) (width 0.5) (layer F.Cu) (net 3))
 (segment (start 127.7 50.55) (end 128.35 50.55) (width 0.5) (layer F.Cu) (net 3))
 (segment (start 128.35 50.55) (end 128.35 149.45) (width 0.5) (layer F.Cu) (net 3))
 (segment (start 128.35 149.45) (end 129 149.45) (width 0.5) (layer F.Cu) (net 3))
 (segment (start 129 50.55) (end 129 149.45) (width 0.5) (layer F.Cu) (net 3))
 (segment (start 129 50.55) (end 129.65 50.55) (width 0.5) (layer F.Cu) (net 3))
 (segment (start 129.65 50.55) (end 129.65 149.45) (width 0.5) (layer F.Cu) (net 3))
 (segment (start 129.65 149.45) (end 130.3 149.45) (width 0.5) (layer F.Cu) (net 3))
 (segment (start 130.3 50.55) (end 130.3 149.45) (width 0.5) (layer F.Cu) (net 3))
 (segment (start 130.3 50.55) (end 130.95 50.55) (width 0.5) (layer F.Cu) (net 3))
 (segment (start 130.95 50.55) (end 130.95 149.45) (width 0.5) (layer F.Cu) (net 3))
 (segment (start 130.95 149.45) (end 131.6 149.45) (width 0.5) (layer F.Cu) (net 3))
 (segment (start 131.6 50.55) (end 131.6 149.45) (width 0.5) (layer F.Cu) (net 3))
 (segment (start 131.6 50.55) (end 132.25 50.55) (width 0.5) (layer F.Cu) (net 3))
 (segment (start 132.25 50.55) (end 132.25 149.45) (width 0.5) (layer F.Cu) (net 3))
 (segment (start 132.25 149.45) (end 132.9 149.45) (width 0.5) (layer F.Cu) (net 3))
 (segment (start 132.9 50.55) (end 132.9 149.45) (width 0.5) (layer F.Cu) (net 3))
 (segment (start 132.9 50.55) (end 133.55 50.55) (width 0.5) (layer F.Cu) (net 3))
 (segment (start 133.55 50.55) (end 133.55 149.45) (width 0.5) (layer F.Cu) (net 3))
 (segment (start 133.55 149.45) (end 134.2 149.45) (width 0.5) (layer F.Cu) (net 3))
 (segment (start 134.2 50.55) (end 134.2 149.45) (width 0.5) (layer F.Cu) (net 3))
 (segment (start 134.2 50.55) (end 134.85 50.55) (width 0.5) (layer F.Cu) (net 3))
 (segment (start 134.85 50.55) (end 134.85 149.45) (width 0.5) (layer F.Cu) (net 3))
 (segment (start 134.85 149.45) (end 135.5 149.45) (width 0.5) (layer F.Cu) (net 3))
 (segment (start 135.5 50.55) (end 135.5 149.45) (width 0.5) (layer F.Cu) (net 3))
 (segment (start 135.5 50.55) (end 136.15 50.55) (width 0.5) (layer F.Cu) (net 3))
 (segment (start 136.15 50.55) (end 136.15 149.45) (width 0.5) (layer F.Cu) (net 3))
 (segment (start 136.15 149.45) (end 136.8 149.45) (width 0.5) (layer F.Cu) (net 3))
 (segment (start 136.8 50.55) (end 136.8 149.45) (width 0.5) (layer F.Cu) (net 3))
 (segment (start 136.8 50.55) (end 137.45 50.55) (width 0.5) (layer F.Cu) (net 3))
 (segment (start 137.45 50.55) (end 137.45 149.45) (width 0.5) (layer F.Cu) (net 3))
 (segment (start 137.45 149.45) (end 138.1 149.45) (width 0.5) (layer F.Cu) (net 3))
 (segment (start 138.1 50.55) (end 138.1 149.45) (width 0.5) (layer F.Cu) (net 3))
 (segment (start 138.1 50.55) (end 138.75 50.55) (width 0.5) (layer F.Cu) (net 3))
 (segment (start 138.75 50.55) (end 138.75 149.45) (width 0.5) (layer F.Cu) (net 3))
 (segment (start 138.75 149.45) (end 139.4 149.45) (width 0.5) (layer F.Cu) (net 3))
 (segment (start 139.4 50.55) (end 139.4 149.45) (width 0.5) (layer F.Cu) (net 3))
 (segment (start 139.4 50.55) (end 140.05 50.55) (width 0.5) (layer F.Cu) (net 3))
 (segment (start 140.05 50.55) (end 140.05 149.45) (width 0.5) (layer F.Cu) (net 3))
 (segment (start 140.05 149.45) (end 140.7 149.45) (width 0.5) (layer F.Cu) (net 3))
 (segment (start 140.7 50.55) (end 140.7 149.45) (width 0.5) (layer F.Cu) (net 3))
 (segment (start 140.7 50.55) (end 141.35 50.55) (width 0.5) (layer F.Cu) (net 3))
 (segment (start 141.35 50.55) (end 141.35 149.45) (width 0.5) (layer F.Cu) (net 3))
 (segment (start 141.35 149.45) (end 142 149.45) (width 0.5) (layer F.Cu) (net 3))
 (segment (start 142 57.75) (end 142 149.45) (width 0.5) (layer F.Cu) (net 3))
 (segment (start 142 57.75) (end 142.65 57.75) (width 0.5) (layer F.Cu) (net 3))
 (segment (start 142.65 57.75) (end 142.65 142.25) (width 0.5) (layer F.Cu) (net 3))
 (segment (start 142.65 142.25) (end 143.3 142.25) (width 0.5) (layer F.Cu) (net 3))
 (segment (start 143.3 57.75) (end 143.3 142.25) (width 0.5) (layer F.Cu) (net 3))
 (segment (start 143.3 57.75) (end 143.95 57.75) (width 0.5) (layer F.Cu) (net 3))
 (segment (start 143.95 57.75) (end 143.95 142.25) (width 0.5) (layer F.Cu) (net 3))
 (segment (start 143.95 142.25) (end 144.6 142.25) (width 0.5) (layer F.Cu) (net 3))
 (segment (start 144.6 57.75) (end 144.6 142.25) (width 0.5) (layer F.Cu) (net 3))
 (segment (start 144.6 57.75) (end 145.25 57.75) (width 0.5) (layer F.Cu) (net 3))
 (segment (start 145.25 57.75) (end 145.25 142.25) (width 0.5) (layer F.Cu) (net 3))
 (segment (start 145.25 142.25) (end 145.9 142.25) (width 0.5) (layer F.Cu) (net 3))
 (segment (start 145.9 57.75) (end 145.9 142.25) (width 0.5) (layer F.Cu) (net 3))
 (segment (start 145.9 57.75) (end 146.55 57.75) (width 0.5) (layer F.Cu) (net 3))
 (segment (start 146.55 57.75) (end 146.55 142.25) (width 0.5) (layer F.Cu) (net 3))
 (segment (start 146.55 142.25) (end 147.2 142.25) (width 0.5) (layer F.Cu) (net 3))
 (segment (start 147.2 57.75) (end 147.2 142.25) (width 0.5) (layer F.Cu) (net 3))
 (segment (start 147.2 57.75) (end 147.85 57.75) (width 0.5) (layer F.Cu) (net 3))
 (segment (start 147.85 57.75) (end 147.85 142.25) (width 0.5) (layer F.Cu) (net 3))
 (segment (start 147.85 142.25) (end 148.5 142.25) (width 0.5) (layer F.Cu) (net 3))
 (segment (start 148.5 57.75) (end 148.5 142.25) (width 0.5) (layer F.Cu) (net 3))
 (segment (start 51.3 142.25) (end 50.65 142.25) (width 0.5) (layer F.Cu) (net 3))
 (segment (start 51.95 142.25) (end 51.95 57.75) (width 0.5) (layer F.Cu) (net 3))
 (segment (start 52.6 57.75) (end 52.6 142.25) (width 0.5) (layer F.Cu) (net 3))
 (segment (start 53.9 142.25) (end 53.25 142.25) (width 0.5) (layer F.Cu) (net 3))
 (segment (start 53.9 57.75) (end 53.9 142.25) (width 0.5) (layer F.Cu) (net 3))
 (segment (start 54.55 142.25) (end 54.55 57.75) (width 0.5) (layer F.Cu) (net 3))
 (segment (start 55.2 57.75) (end 55.2 142.25) (width 0.5) (layer F.Cu) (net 3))
 (segment (start 55.85 57.75) (end 55.2 57.75) (width 0.5) (layer F.Cu) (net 3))
 (segment (start 56.5 57.75) (end 56.5 142.25) (width 0.5) (layer F.Cu) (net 3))
 (segment (start 57.15 57.75) (end 56.5 57.75) (width 0.5) (layer F.Cu) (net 3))
 (segment (start 57.15 142.25) (end 57.15 57.75) (width 0.5) (layer F.Cu) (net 3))
 (segment (start 57.8 50.55) (end 57.8 142.25) (width 0.5) (layer F.Cu) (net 3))
 (segment (start 58.45 50.55) (end 57.8 50.55) (width 0.5) (layer F.Cu) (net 3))
 (segment (start 58.45 149.45) (end 58.45 50.55) (width 0.5) (layer F.Cu) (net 3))
 (segment (start 59.1 149.45) (end 58.45 149.45) (width 0.5) (layer F.Cu) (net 3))
 (segment (start 59.1 50.55) (end 59.1 149.45) (width 0.5) (layer F.Cu) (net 3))
 (segment (start 60.4 149.45) (end 59.75 149.45) (width 0.5) (layer F.Cu) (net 3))
 (segment (start 60.4 50.55) (end 60.4 149.45) (width 0.5) (layer F.Cu) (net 3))
 (segment (start 61.05 50.55) (end 60.4 50.55) (width 0.5) (layer F.Cu) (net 3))
 (segment (start 61.05 149.45) (end 61.05 50.55) (width 0.5) (layer F.Cu) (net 3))
 (segment (start 61.7 149.45) (end 61.05 149.45) (width 0.5) (layer F.Cu) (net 3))
 (segment (start 62.35 50.55) (end 61.7 50.55) (width 0.5) (layer F.Cu) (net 3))
 (segment (start 62.35 149.45) (end 62.35 50.55) (width 0.5) (layer F.Cu) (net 3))
 (segment (start 63 149.45) (end 62.35 149.45) (width 0.5) (layer F.Cu) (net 3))
 (segment (start 63 50.55) (end 63 149.45) (width 0.5) (layer F.Cu) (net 3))
 (segment (start 63.65 50.55) (end 63 50.55) (width 0.5) (layer F.Cu) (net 3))
 (segment (start 75.35 50.55) (end 74.7 50.55) (width 0.5) (layer F.Cu) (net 3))
 (segment (start 76 50.55) (end 76 149.45) (width 0.5) (layer F.Cu) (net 3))
 (segment (start 76.65 50.55) (end 76 50.55) (width 0.5) (layer F.Cu) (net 3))
 (segment (start 76.65 149.45) (end 76.65 50.55) (width 0.5) (layer F.Cu) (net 3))
 (segment (start 77.3 149.45) (end 76.65 149.45) (width 0.5) (layer F.Cu) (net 3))
 (segment (start 66.9 149.45) (end 66.25 149.45) (width 0.5) (layer F.Cu) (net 3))
 (segment (start 74.05 149.45) (end 74.05 50.55) (width 0.5) (layer F.Cu) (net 3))
 (segment (start 54.55 57.75) (end 53.9 57.75) (width 0.5) (layer F.Cu) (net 3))
 (segment (start 73.4 50.55) (end 73.4 149.45) (width 0.5) (layer F.Cu) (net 3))
 (segment (start 78.6 50.55) (end 78.6 149.45) (width 0.5) (layer F.Cu) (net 3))
 (segment (start 76 149.45) (end 75.35 149.45) (width 0.5) (layer F.Cu) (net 3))
 (segment (start 59.75 50.55) (end 59.1 50.55) (width 0.5) (layer F.Cu) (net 3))
 (segment (start 71.45 50.55) (end 70.8 50.55) (width 0.5) (layer F.Cu) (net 3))
 (segment (start 66.25 149.45) (end 66.25 50.55) (width 0.5) (layer F.Cu) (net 3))
 (segment (start 65.6 50.55) (end 65.6 149.45) (width 0.5) (layer F.Cu) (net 3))
 (segment (start 77.95 149.45) (end 77.95 50.55) (width 0.5) (layer F.Cu) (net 3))
 (segment (start 57.8 142.25) (end 57.15 142.25) (width 0.5) (layer F.Cu) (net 3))
 (segment (start 72.1 149.45) (end 71.45 149.45) (width 0.5) (layer F.Cu) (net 3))
 (segment (start 78.6 149.45) (end 77.95 149.45) (width 0.5) (layer F.Cu) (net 3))
 (segment (start 50.65 57.05) (end 50.7 57) (width 0.5) (layer F.Cu) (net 3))
 (segment (start 68.2 50.55) (end 68.2 149.45) (width 0.5) (layer F.Cu) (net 3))
 (segment (start 82.5 50.55) (end 82.5 149.45) (width 0.5) (layer F.Cu) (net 3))
 (segment (start 82.5 149.45) (end 81.85 149.45) (width 0.5) (layer F.Cu) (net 3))
 (segment (start 51.3 57.75) (end 51.3 142.25) (width 0.5) (layer F.Cu) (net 3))
 (segment (start 74.05 50.55) (end 73.4 50.55) (width 0.5) (layer F.Cu) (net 3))
 (segment (start 79.25 149.45) (end 79.25 50.55) (width 0.5) (layer F.Cu) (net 3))
 (segment (start 81.85 50.55) (end 81.2 50.55) (width 0.5) (layer F.Cu) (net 3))
 (segment (start 66.9 50.55) (end 66.9 149.45) (width 0.5) (layer F.Cu) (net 3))
 (segment (start 74.7 50.55) (end 74.7 149.45) (width 0.5) (layer F.Cu) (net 3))
 (segment (start 81.2 149.45) (end 80.55 149.45) (width 0.5) (layer F.Cu) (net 3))
 (segment (start 81.2 50.55) (end 81.2 149.45) (width 0.5) (layer F.Cu) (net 3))
 (segment (start 56.5 142.25) (end 55.85 142.25) (width 0.5) (layer F.Cu) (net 3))
 (segment (start 73.4 149.45) (end 72.75 149.45) (width 0.5) (layer F.Cu) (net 3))
 (segment (start 75.35 149.45) (end 75.35 50.55) (width 0.5) (layer F.Cu) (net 3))
 (segment (start 80.55 149.45) (end 80.55 50.55) (width 0.5) (layer F.Cu) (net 3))
 (segment (start 81.85 149.45) (end 81.85 50.55) (width 0.5) (layer F.Cu) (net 3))
 (segment (start 74.7 149.45) (end 74.05 149.45) (width 0.5) (layer F.Cu) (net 3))
 (segment (start 80.55 50.55) (end 79.9 50.55) (width 0.5) (layer F.Cu) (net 3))
 (segment (start 77.3 50.55) (end 77.3 149.45) (width 0.5) (layer F.Cu) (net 3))
 (segment (start 63.65 149.45) (end 63.65 50.55) (width 0.5) (layer F.Cu) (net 3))
 (segment (start 79.9 50.55) (end 79.9 149.45) (width 0.5) (layer F.Cu) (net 3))
 (segment (start 64.3 149.45) (end 63.65 149.45) (width 0.5) (layer F.Cu) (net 3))
 (segment (start 71.45 149.45) (end 71.45 50.55) (width 0.5) (layer F.Cu) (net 3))
 (segment (start 79.9 149.45) (end 79.25 149.45) (width 0.5) (layer F.Cu) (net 3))
 (segment (start 70.8 149.45) (end 70.15 149.45) (width 0.5) (layer F.Cu) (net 3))
 (segment (start 79.25 50.55) (end 78.6 50.55) (width 0.5) (layer F.Cu) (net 3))
 (segment (start 59.75 149.45) (end 59.75 50.55) (width 0.5) (layer F.Cu) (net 3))
 (segment (start 72.75 149.45) (end 72.75 50.55) (width 0.5) (layer F.Cu) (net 3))
 (segment (start 64.95 149.45) (end 64.95 50.55) (width 0.5) (layer F.Cu) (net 3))
 (segment (start 72.75 50.55) (end 72.1 50.55) (width 0.5) (layer F.Cu) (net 3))
 (segment (start 66.25 50.55) (end 65.6 50.55) (width 0.5) (layer F.Cu) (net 3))
 (segment (start 72.1 50.55) (end 72.1 149.45) (width 0.5) (layer F.Cu) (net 3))
 (segment (start 53.25 142.25) (end 53.25 57.75) (width 0.5) (layer F.Cu) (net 3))
 (segment (start 70.8 50.55) (end 70.8 149.45) (width 0.5) (layer F.Cu) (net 3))
 (segment (start 77.95 50.55) (end 77.3 50.55) (width 0.5) (layer F.Cu) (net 3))
 (segment (start 64.95 50.55) (end 64.3 50.55) (width 0.5) (layer F.Cu) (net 3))
 (segment (start 70.15 149.45) (end 70.15 50.55) (width 0.5) (layer F.Cu) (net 3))
 (segment (start 55.2 142.25) (end 54.55 142.25) (width 0.5) (layer F.Cu) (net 3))
 (segment (start 70.15 50.55) (end 69.5 50.55) (width 0.5) (layer F.Cu) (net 3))
 (segment (start 53.25 57.75) (end 52.6 57.75) (width 0.5) (layer F.Cu) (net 3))
 (segment (start 69.5 50.55) (end 69.5 149.45) (width 0.5) (layer F.Cu) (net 3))
 (segment (start 55.85 142.25) (end 55.85 57.75) (width 0.5) (layer F.Cu) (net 3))
 (segment (start 69.5 149.45) (end 68.85 149.45) (width 0.5) (layer F.Cu) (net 3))
 (segment (start 61.7 50.55) (end 61.7 149.45) (width 0.5) (layer F.Cu) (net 3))
 (segment (start 68.85 149.45) (end 68.85 50.55) (width 0.5) (layer F.Cu) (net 3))
 (segment (start 51.95 57.75) (end 51.3 57.75) (width 0.5) (layer F.Cu) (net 3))
 (segment (start 68.85 50.55) (end 68.2 50.55) (width 0.5) (layer F.Cu) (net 3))
 (segment (start 52.6 142.25) (end 51.95 142.25) (width 0.5) (layer F.Cu) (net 3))
 (segment (start 68.2 149.45) (end 67.55 149.45) (width 0.5) (layer F.Cu) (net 3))
 (segment (start 64.3 50.55) (end 64.3 149.45) (width 0.5) (layer F.Cu) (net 3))
 (segment (start 50.65 142.25) (end 50.65 57.05) (width 0.5) (layer F.Cu) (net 3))
 (segment (start 67.55 149.45) (end 67.55 50.55) (width 0.5) (layer F.Cu) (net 3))
 (segment (start 67.55 50.55) (end 66.9 50.55) (width 0.5) (layer F.Cu) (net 3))
 (segment (start 65.6 149.45) (end 64.95 149.45) (width 0.5) (layer F.Cu) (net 3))
 (segment (start 148.55 56.95) (end 148.55 58.15) (width 0.6) (layer F.Cu) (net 3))
 (segment (start 148.55 58.25) (end 148.4 58.4) (width 1) (layer B.Cu) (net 3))
 (segment (start 148.55 56.95) (end 148.55 58.25) (width 1) (layer B.Cu) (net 3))
 (segment (start 105.4 58.4) (end 148.4 58.4) (width 1) (layer B.Cu) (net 3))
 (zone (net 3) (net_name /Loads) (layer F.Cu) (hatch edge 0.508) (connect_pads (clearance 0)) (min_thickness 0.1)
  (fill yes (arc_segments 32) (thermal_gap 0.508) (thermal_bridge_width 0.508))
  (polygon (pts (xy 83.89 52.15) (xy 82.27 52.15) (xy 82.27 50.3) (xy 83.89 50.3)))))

